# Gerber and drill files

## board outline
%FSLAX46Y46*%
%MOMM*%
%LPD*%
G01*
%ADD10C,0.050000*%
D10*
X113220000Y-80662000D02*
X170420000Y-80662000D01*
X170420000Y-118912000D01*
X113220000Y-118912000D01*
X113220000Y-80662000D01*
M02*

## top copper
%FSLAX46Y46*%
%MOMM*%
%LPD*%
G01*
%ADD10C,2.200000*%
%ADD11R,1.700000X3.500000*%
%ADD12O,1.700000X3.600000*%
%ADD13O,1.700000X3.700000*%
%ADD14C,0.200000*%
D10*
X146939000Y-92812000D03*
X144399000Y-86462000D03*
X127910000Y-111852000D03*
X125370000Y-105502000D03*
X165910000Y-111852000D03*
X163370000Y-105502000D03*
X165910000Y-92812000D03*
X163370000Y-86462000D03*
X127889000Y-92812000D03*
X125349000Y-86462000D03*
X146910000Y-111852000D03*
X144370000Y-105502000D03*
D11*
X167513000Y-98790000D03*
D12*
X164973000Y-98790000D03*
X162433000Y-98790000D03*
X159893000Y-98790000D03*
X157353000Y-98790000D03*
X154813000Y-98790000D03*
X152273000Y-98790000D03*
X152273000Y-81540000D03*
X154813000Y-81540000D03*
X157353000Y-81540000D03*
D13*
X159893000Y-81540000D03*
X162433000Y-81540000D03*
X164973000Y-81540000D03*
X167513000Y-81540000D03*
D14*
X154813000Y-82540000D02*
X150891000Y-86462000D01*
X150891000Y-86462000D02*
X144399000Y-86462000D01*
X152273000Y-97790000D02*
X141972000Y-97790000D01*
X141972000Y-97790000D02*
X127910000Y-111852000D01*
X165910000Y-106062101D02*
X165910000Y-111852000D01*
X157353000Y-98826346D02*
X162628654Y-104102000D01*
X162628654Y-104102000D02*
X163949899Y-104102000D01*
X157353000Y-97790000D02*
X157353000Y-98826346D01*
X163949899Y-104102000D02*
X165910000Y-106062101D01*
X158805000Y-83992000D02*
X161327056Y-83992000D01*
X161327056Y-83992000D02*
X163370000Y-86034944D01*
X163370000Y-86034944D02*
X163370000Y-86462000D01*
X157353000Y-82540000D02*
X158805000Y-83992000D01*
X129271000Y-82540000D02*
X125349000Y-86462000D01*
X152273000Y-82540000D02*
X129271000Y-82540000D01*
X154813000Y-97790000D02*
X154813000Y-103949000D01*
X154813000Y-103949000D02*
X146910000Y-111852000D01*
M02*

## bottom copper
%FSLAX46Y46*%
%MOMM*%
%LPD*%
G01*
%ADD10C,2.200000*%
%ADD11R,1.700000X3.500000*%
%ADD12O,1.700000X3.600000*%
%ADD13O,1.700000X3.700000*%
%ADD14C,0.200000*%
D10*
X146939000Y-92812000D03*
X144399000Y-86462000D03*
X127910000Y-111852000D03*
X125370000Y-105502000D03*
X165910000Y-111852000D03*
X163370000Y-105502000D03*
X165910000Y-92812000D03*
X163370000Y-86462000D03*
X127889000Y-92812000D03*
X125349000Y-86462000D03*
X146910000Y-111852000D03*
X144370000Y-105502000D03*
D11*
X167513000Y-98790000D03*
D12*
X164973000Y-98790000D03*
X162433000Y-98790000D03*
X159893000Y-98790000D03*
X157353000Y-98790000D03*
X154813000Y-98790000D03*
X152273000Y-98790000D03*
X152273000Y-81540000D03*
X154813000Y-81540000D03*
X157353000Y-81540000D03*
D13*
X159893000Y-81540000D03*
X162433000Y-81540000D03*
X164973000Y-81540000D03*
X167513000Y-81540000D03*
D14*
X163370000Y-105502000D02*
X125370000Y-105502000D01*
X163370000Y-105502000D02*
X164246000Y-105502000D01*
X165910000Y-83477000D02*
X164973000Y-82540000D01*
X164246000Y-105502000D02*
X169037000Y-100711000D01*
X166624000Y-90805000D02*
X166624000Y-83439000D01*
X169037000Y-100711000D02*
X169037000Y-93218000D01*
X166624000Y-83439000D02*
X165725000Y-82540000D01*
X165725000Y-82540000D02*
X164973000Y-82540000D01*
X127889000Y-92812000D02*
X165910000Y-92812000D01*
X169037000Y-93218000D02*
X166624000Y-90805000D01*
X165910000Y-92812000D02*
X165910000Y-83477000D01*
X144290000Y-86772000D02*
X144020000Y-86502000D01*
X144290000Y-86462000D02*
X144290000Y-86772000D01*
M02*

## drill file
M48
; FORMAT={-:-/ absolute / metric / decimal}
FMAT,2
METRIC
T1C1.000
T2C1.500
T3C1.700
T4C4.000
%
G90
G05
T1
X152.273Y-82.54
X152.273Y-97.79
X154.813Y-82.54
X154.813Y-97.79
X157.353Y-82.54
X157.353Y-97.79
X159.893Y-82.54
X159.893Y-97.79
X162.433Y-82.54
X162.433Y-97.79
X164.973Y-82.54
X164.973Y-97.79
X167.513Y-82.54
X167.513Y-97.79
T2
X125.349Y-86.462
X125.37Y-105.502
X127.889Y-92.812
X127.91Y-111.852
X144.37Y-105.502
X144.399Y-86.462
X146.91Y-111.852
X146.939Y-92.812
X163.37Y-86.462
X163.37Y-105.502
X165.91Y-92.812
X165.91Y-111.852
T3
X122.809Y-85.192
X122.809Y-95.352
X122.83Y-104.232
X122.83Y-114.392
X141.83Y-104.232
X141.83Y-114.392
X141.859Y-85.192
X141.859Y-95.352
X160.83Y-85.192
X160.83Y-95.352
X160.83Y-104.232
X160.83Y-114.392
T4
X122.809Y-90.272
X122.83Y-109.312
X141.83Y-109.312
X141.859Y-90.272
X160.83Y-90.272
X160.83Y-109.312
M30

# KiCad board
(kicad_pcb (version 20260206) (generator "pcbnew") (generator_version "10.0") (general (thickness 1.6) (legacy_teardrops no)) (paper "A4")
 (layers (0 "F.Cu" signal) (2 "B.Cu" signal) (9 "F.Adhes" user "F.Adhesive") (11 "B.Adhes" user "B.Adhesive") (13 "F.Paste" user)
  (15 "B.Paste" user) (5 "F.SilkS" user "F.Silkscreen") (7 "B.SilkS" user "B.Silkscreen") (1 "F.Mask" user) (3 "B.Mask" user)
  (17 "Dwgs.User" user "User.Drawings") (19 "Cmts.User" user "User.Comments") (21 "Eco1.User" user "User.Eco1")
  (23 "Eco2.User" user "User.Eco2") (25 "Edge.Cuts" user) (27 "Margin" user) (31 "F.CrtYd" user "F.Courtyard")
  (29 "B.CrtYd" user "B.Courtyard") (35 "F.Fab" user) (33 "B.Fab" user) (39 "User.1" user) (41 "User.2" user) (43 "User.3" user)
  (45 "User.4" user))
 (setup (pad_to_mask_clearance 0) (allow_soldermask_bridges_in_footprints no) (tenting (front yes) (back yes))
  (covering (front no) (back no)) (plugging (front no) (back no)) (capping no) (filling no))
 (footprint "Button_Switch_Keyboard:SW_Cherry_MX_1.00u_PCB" (layer "F.Cu") (at 146.939 92.812 -90)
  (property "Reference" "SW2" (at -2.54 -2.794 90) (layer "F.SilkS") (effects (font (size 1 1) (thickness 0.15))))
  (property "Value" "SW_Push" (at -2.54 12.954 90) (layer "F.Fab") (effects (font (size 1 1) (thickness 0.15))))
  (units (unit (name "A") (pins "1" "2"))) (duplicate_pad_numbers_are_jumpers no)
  (pad "" np_thru_hole circle (at -7.62 5.08 270) (size 1.7 1.7) (drill 1.7) (layers "*.Cu" "*.Mask"))
  (pad "" np_thru_hole circle (at -2.54 5.08 270) (size 4 4) (drill 4) (layers "*.Cu" "*.Mask"))
  (pad "" np_thru_hole circle (at 2.54 5.08 270) (size 1.7 1.7) (drill 1.7) (layers "*.Cu" "*.Mask"))
  (pad "1" thru_hole circle (at 0 0 270) (size 2.2 2.2) (drill 1.5) (layers "*.Cu" "*.Mask") (remove_unused_layers no) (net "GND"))
  (pad "2" thru_hole circle (at -6.35 2.54 270) (size 2.2 2.2) (drill 1.5) (layers "*.Cu" "*.Mask") (remove_unused_layers no)
   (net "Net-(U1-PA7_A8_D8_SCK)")))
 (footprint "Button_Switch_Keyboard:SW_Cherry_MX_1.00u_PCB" (layer "F.Cu") (at 127.91 111.852 -90)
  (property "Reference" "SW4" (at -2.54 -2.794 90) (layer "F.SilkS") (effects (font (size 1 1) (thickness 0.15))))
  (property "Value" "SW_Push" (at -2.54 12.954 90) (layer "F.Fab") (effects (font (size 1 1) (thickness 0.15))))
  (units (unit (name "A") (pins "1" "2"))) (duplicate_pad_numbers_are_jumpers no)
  (pad "" np_thru_hole circle (at -7.62 5.08 270) (size 1.7 1.7) (drill 1.7) (layers "*.Cu" "*.Mask"))
  (pad "" np_thru_hole circle (at -2.54 5.08 270) (size 4 4) (drill 4) (layers "*.Cu" "*.Mask"))
  (pad "" np_thru_hole circle (at 2.54 5.08 270) (size 1.7 1.7) (drill 1.7) (layers "*.Cu" "*.Mask"))
  (pad "1" thru_hole circle (at 0 0 270) (size 2.2 2.2) (drill 1.5) (layers "*.Cu" "*.Mask") (remove_unused_layers no)
   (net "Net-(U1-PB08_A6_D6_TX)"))
  (pad "2" thru_hole circle (at -6.35 2.54 270) (size 2.2 2.2) (drill 1.5) (layers "*.Cu" "*.Mask") (remove_unused_layers no) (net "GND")))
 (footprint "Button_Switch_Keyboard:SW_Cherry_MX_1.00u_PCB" (layer "F.Cu") (at 165.91 111.852 -90)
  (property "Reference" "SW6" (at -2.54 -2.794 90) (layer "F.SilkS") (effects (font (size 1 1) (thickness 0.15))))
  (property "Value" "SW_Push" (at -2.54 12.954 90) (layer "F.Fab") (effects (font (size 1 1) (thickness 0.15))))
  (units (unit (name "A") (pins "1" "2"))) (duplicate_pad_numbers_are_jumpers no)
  (pad "" np_thru_hole circle (at -7.62 5.08 270) (size 1.7 1.7) (drill 1.7) (layers "*.Cu" "*.Mask"))
  (pad "" np_thru_hole circle (at -2.54 5.08 270) (size 4 4) (drill 4) (layers "*.Cu" "*.Mask"))
  (pad "" np_thru_hole circle (at 2.54 5.08 270) (size 1.7 1.7) (drill 1.7) (layers "*.Cu" "*.Mask"))
  (pad "1" thru_hole circle (at 0 0 270) (size 2.2 2.2) (drill 1.5) (layers "*.Cu" "*.Mask") (remove_unused_layers no)
   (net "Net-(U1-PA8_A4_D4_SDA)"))
  (pad "2" thru_hole circle (at -6.35 2.54 270) (size 2.2 2.2) (drill 1.5) (layers "*.Cu" "*.Mask") (remove_unused_layers no) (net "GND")))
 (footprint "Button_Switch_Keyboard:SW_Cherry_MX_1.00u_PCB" (layer "F.Cu") (at 165.91 92.812 -90)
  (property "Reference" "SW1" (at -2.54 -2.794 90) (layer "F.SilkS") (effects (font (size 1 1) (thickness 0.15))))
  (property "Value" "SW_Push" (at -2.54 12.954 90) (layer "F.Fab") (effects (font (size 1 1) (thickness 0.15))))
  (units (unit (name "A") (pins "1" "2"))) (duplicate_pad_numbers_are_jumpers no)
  (pad "" np_thru_hole circle (at -7.62 5.08 270) (size 1.7 1.7) (drill 1.7) (layers "*.Cu" "*.Mask"))
  (pad "" np_thru_hole circle (at -2.54 5.08 270) (size 4 4) (drill 4) (layers "*.Cu" "*.Mask"))
  (pad "" np_thru_hole circle (at 2.54 5.08 270) (size 1.7 1.7) (drill 1.7) (layers "*.Cu" "*.Mask"))
  (pad "1" thru_hole circle (at 0 0 270) (size 2.2 2.2) (drill 1.5) (layers "*.Cu" "*.Mask") (remove_unused_layers no) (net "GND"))
  (pad "2" thru_hole circle (at -6.35 2.54 270) (size 2.2 2.2) (drill 1.5) (layers "*.Cu" "*.Mask") (remove_unused_layers no)
   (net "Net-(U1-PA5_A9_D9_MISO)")))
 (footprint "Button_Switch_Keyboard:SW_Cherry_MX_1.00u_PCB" (layer "F.Cu") (at 127.889 92.812 -90)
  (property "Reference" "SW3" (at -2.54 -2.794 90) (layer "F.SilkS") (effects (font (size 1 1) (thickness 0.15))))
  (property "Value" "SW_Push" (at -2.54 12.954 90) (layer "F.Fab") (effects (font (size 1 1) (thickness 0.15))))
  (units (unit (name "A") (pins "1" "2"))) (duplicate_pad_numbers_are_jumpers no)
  (pad "" np_thru_hole circle (at -7.62 5.08 270) (size 1.7 1.7) (drill 1.7) (layers "*.Cu" "*.Mask"))
  (pad "" np_thru_hole circle (at -2.54 5.08 270) (size 4 4) (drill 4) (layers "*.Cu" "*.Mask"))
  (pad "" np_thru_hole circle (at 2.54 5.08 270) (size 1.7 1.7) (drill 1.7) (layers "*.Cu" "*.Mask"))
  (pad "1" thru_hole circle (at 0 0 270) (size 2.2 2.2) (drill 1.5) (layers "*.Cu" "*.Mask") (remove_unused_layers no) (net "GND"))
  (pad "2" thru_hole circle (at -6.35 2.54 270) (size 2.2 2.2) (drill 1.5) (layers "*.Cu" "*.Mask") (remove_unused_layers no)
   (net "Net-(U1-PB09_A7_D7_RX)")))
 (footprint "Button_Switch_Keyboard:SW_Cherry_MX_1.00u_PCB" (layer "F.Cu") (at 146.91 111.852 -90)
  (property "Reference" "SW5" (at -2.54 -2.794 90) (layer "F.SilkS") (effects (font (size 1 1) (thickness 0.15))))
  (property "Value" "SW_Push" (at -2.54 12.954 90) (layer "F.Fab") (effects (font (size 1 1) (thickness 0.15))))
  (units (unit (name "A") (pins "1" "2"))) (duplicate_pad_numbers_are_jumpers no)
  (pad "" np_thru_hole circle (at -7.62 5.08 270) (size 1.7 1.7) (drill 1.7) (layers "*.Cu" "*.Mask"))
  (pad "" np_thru_hole circle (at -2.54 5.08 270) (size 4 4) (drill 4) (layers "*.Cu" "*.Mask"))
  (pad "" np_thru_hole circle (at 2.54 5.08 270) (size 1.7 1.7) (drill 1.7) (layers "*.Cu" "*.Mask"))
  (pad "1" thru_hole circle (at 0 0 270) (size 2.2 2.2) (drill 1.5) (layers "*.Cu" "*.Mask") (remove_unused_layers no)
   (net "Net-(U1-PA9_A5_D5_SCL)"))
  (pad "2" thru_hole circle (at -6.35 2.54 270) (size 2.2 2.2) (drill 1.5) (layers "*.Cu" "*.Mask") (remove_unused_layers no) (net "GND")))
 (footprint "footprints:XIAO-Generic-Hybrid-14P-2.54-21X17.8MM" (layer "B.Cu") (at 159.893 90.165 90)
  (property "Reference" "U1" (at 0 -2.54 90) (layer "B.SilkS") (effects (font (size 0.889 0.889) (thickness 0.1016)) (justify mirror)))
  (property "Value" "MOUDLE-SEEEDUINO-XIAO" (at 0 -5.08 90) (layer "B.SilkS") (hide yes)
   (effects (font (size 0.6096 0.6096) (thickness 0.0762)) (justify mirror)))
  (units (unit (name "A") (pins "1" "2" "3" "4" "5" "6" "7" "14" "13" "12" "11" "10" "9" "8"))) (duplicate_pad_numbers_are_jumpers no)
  (pad "1" thru_hole rect (at -7.625 7.62 90) (size 3.5 1.7) (drill 1 (offset -1 0)) (layers "*.Cu" "*.Mask") (remove_unused_layers no)
   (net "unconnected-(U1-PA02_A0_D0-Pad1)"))
  (pad "2" thru_hole oval (at -7.625 5.08 90) (size 3.6 1.7) (drill 1 (offset -1 0)) (layers "*.Cu" "*.Mask") (remove_unused_layers no)
   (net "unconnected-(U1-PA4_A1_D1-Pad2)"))
  (pad "3" thru_hole oval (at -7.625 2.54 90) (size 3.6 1.7) (drill 1 (offset -1 0)) (layers "*.Cu" "*.Mask") (remove_unused_layers no)
   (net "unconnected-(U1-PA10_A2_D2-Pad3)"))
  (pad "4" thru_hole oval (at -7.625 0 90) (size 3.6 1.7) (drill 1 (offset -1 0)) (layers "*.Cu" "*.Mask") (remove_unused_layers no)
   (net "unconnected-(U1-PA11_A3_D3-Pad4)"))
  (pad "5" thru_hole oval (at -7.625 -2.54 90) (size 3.6 1.7) (drill 1 (offset -1 0)) (layers "*.Cu" "*.Mask") (remove_unused_layers no)
   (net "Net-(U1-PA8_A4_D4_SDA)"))
  (pad "6" thru_hole oval (at -7.625 -5.08 270) (size 3.6 1.7) (drill 1 (offset 1 0)) (layers "*.Cu" "*.Mask") (remove_unused_layers no)
   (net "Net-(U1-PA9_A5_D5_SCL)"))
  (pad "7" thru_hole oval (at -7.625 -7.62 90) (size 3.6 1.7) (drill 1 (offset -1 0)) (layers "*.Cu" "*.Mask") (remove_unused_layers no)
   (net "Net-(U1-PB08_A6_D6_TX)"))
  (pad "8" thru_hole oval (at 7.625 -7.62 90) (size 3.6 1.7) (drill 1 (offset 1 0)) (layers "*.Cu" "*.Mask") (remove_unused_layers no)
   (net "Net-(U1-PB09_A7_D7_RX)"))
  (pad "9" thru_hole oval (at 7.625 -5.08 90) (size 3.6 1.7) (drill 1 (offset 1 0)) (layers "*.Cu" "*.Mask") (remove_unused_layers no)
   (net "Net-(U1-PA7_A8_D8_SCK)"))
  (pad "10" thru_hole oval (at 7.625 -2.54 90) (size 3.6 1.7) (drill 1 (offset 1 0)) (layers "*.Cu" "*.Mask") (remove_unused_layers no)
   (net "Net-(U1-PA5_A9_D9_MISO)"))
  (pad "11" thru_hole oval (at 7.625 0 90) (size 3.7 1.7) (drill 1 (offset 1 0)) (layers "*.Cu" "*.Mask") (remove_unused_layers no)
   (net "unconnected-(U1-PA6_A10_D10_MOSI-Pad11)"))
  (pad "12" thru_hole oval (at 7.625 2.54 90) (size 3.7 1.7) (drill 1 (offset 1 0)) (layers "*.Cu" "*.Mask") (remove_unused_layers no)
   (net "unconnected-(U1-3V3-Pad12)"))
  (pad "13" thru_hole oval (at 7.625 5.08 90) (size 3.7 1.7) (drill 1 (offset 1 0)) (layers "*.Cu" "*.Mask") (remove_unused_layers no)
   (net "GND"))
  (pad "14" thru_hole oval (at 7.625 7.62 90) (size 3.7 1.7) (drill 1 (offset 1 0)) (layers "*.Cu" "*.Mask") (remove_unused_layers no)
   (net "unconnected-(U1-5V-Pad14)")))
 (gr_rect (start 113.22 80.662) (end 170.42 118.912) (stroke (width 0.05) (type default)) (fill no) (layer "Edge.Cuts"))
 (segment (start 163.37 105.502) (end 125.37 105.502) (width 0.2) (layer "B.Cu") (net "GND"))
 (segment (start 163.37 105.502) (end 164.246 105.502) (width 0.2) (layer "B.Cu") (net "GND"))
 (segment (start 165.91 83.477) (end 164.973 82.54) (width 0.2) (layer "B.Cu") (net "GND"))
 (segment (start 164.246 105.502) (end 169.037 100.711) (width 0.2) (layer "B.Cu") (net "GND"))
 (segment (start 166.624 90.805) (end 166.624 83.439) (width 0.2) (layer "B.Cu") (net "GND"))
 (segment (start 169.037 100.711) (end 169.037 93.218) (width 0.2) (layer "B.Cu") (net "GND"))
 (segment (start 166.624 83.439) (end 165.725 82.54) (width 0.2) (layer "B.Cu") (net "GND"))
 (segment (start 165.725 82.54) (end 164.973 82.54) (width 0.2) (layer "B.Cu") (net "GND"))
 (segment (start 127.889 92.812) (end 165.91 92.812) (width 0.2) (layer "B.Cu") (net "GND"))
 (segment (start 169.037 93.218) (end 166.624 90.805) (width 0.2) (layer "B.Cu") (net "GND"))
 (segment (start 165.91 92.812) (end 165.91 83.477) (width 0.2) (layer "B.Cu") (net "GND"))
 (segment (start 154.813 82.54) (end 150.891 86.462) (width 0.2) (layer "F.Cu") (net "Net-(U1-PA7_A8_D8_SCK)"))
 (segment (start 150.891 86.462) (end 144.399 86.462) (width 0.2) (layer "F.Cu") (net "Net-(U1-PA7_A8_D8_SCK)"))
 (segment (start 144.29 86.772) (end 144.02 86.502) (width 0.2) (layer "B.Cu") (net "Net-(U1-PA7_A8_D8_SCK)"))
 (segment (start 144.29 86.462) (end 144.29 86.772) (width 0.2) (layer "B.Cu") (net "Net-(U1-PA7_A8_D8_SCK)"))
 (segment (start 152.273 97.79) (end 141.972 97.79) (width 0.2) (layer "F.Cu") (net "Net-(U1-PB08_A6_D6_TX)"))
 (segment (start 141.972 97.79) (end 127.91 111.852) (width 0.2) (layer "F.Cu") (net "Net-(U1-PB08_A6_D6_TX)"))
 (segment (start 165.91 106.062101) (end 165.91 111.852) (width 0.2) (layer "F.Cu") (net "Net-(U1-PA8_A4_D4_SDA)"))
 (segment (start 157.353 98.826346) (end 162.628654 104.102) (width 0.2) (layer "F.Cu") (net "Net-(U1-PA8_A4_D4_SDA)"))
 (segment (start 162.628654 104.102) (end 163.949899 104.102) (width 0.2) (layer "F.Cu") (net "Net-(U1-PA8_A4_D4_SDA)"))
 (segment (start 157.353 97.79) (end 157.353 98.826346) (width 0.2) (layer "F.Cu") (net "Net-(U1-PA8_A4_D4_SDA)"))
 (segment (start 163.949899 104.102) (end 165.91 106.062101) (width 0.2) (layer "F.Cu") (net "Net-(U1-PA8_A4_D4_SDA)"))
 (segment (start 158.805 83.992) (end 161.327056 83.992) (width 0.2) (layer "F.Cu") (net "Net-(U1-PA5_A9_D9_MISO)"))
 (segment (start 161.327056 83.992) (end 163.37 86.034944) (width 0.2) (layer "F.Cu") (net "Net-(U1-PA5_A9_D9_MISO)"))
 (segment (start 163.37 86.034944) (end 163.37 86.462) (width 0.2) (layer "F.Cu") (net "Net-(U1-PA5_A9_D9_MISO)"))
 (segment (start 157.353 82.54) (end 158.805 83.992) (width 0.2) (layer "F.Cu") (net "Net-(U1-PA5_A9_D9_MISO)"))
 (segment (start 129.271 82.54) (end 125.349 86.462) (width 0.2) (layer "F.Cu") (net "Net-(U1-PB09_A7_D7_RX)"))
 (segment (start 152.273 82.54) (end 129.271 82.54) (width 0.2) (layer "F.Cu") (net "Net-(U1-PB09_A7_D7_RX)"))
 (segment (start 154.813 97.79) (end 154.813 103.949) (width 0.2) (layer "F.Cu") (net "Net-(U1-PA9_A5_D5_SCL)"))
 (segment (start 154.813 103.949) (end 146.91 111.852) (width 0.2) (layer "F.Cu") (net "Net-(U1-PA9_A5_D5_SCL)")))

